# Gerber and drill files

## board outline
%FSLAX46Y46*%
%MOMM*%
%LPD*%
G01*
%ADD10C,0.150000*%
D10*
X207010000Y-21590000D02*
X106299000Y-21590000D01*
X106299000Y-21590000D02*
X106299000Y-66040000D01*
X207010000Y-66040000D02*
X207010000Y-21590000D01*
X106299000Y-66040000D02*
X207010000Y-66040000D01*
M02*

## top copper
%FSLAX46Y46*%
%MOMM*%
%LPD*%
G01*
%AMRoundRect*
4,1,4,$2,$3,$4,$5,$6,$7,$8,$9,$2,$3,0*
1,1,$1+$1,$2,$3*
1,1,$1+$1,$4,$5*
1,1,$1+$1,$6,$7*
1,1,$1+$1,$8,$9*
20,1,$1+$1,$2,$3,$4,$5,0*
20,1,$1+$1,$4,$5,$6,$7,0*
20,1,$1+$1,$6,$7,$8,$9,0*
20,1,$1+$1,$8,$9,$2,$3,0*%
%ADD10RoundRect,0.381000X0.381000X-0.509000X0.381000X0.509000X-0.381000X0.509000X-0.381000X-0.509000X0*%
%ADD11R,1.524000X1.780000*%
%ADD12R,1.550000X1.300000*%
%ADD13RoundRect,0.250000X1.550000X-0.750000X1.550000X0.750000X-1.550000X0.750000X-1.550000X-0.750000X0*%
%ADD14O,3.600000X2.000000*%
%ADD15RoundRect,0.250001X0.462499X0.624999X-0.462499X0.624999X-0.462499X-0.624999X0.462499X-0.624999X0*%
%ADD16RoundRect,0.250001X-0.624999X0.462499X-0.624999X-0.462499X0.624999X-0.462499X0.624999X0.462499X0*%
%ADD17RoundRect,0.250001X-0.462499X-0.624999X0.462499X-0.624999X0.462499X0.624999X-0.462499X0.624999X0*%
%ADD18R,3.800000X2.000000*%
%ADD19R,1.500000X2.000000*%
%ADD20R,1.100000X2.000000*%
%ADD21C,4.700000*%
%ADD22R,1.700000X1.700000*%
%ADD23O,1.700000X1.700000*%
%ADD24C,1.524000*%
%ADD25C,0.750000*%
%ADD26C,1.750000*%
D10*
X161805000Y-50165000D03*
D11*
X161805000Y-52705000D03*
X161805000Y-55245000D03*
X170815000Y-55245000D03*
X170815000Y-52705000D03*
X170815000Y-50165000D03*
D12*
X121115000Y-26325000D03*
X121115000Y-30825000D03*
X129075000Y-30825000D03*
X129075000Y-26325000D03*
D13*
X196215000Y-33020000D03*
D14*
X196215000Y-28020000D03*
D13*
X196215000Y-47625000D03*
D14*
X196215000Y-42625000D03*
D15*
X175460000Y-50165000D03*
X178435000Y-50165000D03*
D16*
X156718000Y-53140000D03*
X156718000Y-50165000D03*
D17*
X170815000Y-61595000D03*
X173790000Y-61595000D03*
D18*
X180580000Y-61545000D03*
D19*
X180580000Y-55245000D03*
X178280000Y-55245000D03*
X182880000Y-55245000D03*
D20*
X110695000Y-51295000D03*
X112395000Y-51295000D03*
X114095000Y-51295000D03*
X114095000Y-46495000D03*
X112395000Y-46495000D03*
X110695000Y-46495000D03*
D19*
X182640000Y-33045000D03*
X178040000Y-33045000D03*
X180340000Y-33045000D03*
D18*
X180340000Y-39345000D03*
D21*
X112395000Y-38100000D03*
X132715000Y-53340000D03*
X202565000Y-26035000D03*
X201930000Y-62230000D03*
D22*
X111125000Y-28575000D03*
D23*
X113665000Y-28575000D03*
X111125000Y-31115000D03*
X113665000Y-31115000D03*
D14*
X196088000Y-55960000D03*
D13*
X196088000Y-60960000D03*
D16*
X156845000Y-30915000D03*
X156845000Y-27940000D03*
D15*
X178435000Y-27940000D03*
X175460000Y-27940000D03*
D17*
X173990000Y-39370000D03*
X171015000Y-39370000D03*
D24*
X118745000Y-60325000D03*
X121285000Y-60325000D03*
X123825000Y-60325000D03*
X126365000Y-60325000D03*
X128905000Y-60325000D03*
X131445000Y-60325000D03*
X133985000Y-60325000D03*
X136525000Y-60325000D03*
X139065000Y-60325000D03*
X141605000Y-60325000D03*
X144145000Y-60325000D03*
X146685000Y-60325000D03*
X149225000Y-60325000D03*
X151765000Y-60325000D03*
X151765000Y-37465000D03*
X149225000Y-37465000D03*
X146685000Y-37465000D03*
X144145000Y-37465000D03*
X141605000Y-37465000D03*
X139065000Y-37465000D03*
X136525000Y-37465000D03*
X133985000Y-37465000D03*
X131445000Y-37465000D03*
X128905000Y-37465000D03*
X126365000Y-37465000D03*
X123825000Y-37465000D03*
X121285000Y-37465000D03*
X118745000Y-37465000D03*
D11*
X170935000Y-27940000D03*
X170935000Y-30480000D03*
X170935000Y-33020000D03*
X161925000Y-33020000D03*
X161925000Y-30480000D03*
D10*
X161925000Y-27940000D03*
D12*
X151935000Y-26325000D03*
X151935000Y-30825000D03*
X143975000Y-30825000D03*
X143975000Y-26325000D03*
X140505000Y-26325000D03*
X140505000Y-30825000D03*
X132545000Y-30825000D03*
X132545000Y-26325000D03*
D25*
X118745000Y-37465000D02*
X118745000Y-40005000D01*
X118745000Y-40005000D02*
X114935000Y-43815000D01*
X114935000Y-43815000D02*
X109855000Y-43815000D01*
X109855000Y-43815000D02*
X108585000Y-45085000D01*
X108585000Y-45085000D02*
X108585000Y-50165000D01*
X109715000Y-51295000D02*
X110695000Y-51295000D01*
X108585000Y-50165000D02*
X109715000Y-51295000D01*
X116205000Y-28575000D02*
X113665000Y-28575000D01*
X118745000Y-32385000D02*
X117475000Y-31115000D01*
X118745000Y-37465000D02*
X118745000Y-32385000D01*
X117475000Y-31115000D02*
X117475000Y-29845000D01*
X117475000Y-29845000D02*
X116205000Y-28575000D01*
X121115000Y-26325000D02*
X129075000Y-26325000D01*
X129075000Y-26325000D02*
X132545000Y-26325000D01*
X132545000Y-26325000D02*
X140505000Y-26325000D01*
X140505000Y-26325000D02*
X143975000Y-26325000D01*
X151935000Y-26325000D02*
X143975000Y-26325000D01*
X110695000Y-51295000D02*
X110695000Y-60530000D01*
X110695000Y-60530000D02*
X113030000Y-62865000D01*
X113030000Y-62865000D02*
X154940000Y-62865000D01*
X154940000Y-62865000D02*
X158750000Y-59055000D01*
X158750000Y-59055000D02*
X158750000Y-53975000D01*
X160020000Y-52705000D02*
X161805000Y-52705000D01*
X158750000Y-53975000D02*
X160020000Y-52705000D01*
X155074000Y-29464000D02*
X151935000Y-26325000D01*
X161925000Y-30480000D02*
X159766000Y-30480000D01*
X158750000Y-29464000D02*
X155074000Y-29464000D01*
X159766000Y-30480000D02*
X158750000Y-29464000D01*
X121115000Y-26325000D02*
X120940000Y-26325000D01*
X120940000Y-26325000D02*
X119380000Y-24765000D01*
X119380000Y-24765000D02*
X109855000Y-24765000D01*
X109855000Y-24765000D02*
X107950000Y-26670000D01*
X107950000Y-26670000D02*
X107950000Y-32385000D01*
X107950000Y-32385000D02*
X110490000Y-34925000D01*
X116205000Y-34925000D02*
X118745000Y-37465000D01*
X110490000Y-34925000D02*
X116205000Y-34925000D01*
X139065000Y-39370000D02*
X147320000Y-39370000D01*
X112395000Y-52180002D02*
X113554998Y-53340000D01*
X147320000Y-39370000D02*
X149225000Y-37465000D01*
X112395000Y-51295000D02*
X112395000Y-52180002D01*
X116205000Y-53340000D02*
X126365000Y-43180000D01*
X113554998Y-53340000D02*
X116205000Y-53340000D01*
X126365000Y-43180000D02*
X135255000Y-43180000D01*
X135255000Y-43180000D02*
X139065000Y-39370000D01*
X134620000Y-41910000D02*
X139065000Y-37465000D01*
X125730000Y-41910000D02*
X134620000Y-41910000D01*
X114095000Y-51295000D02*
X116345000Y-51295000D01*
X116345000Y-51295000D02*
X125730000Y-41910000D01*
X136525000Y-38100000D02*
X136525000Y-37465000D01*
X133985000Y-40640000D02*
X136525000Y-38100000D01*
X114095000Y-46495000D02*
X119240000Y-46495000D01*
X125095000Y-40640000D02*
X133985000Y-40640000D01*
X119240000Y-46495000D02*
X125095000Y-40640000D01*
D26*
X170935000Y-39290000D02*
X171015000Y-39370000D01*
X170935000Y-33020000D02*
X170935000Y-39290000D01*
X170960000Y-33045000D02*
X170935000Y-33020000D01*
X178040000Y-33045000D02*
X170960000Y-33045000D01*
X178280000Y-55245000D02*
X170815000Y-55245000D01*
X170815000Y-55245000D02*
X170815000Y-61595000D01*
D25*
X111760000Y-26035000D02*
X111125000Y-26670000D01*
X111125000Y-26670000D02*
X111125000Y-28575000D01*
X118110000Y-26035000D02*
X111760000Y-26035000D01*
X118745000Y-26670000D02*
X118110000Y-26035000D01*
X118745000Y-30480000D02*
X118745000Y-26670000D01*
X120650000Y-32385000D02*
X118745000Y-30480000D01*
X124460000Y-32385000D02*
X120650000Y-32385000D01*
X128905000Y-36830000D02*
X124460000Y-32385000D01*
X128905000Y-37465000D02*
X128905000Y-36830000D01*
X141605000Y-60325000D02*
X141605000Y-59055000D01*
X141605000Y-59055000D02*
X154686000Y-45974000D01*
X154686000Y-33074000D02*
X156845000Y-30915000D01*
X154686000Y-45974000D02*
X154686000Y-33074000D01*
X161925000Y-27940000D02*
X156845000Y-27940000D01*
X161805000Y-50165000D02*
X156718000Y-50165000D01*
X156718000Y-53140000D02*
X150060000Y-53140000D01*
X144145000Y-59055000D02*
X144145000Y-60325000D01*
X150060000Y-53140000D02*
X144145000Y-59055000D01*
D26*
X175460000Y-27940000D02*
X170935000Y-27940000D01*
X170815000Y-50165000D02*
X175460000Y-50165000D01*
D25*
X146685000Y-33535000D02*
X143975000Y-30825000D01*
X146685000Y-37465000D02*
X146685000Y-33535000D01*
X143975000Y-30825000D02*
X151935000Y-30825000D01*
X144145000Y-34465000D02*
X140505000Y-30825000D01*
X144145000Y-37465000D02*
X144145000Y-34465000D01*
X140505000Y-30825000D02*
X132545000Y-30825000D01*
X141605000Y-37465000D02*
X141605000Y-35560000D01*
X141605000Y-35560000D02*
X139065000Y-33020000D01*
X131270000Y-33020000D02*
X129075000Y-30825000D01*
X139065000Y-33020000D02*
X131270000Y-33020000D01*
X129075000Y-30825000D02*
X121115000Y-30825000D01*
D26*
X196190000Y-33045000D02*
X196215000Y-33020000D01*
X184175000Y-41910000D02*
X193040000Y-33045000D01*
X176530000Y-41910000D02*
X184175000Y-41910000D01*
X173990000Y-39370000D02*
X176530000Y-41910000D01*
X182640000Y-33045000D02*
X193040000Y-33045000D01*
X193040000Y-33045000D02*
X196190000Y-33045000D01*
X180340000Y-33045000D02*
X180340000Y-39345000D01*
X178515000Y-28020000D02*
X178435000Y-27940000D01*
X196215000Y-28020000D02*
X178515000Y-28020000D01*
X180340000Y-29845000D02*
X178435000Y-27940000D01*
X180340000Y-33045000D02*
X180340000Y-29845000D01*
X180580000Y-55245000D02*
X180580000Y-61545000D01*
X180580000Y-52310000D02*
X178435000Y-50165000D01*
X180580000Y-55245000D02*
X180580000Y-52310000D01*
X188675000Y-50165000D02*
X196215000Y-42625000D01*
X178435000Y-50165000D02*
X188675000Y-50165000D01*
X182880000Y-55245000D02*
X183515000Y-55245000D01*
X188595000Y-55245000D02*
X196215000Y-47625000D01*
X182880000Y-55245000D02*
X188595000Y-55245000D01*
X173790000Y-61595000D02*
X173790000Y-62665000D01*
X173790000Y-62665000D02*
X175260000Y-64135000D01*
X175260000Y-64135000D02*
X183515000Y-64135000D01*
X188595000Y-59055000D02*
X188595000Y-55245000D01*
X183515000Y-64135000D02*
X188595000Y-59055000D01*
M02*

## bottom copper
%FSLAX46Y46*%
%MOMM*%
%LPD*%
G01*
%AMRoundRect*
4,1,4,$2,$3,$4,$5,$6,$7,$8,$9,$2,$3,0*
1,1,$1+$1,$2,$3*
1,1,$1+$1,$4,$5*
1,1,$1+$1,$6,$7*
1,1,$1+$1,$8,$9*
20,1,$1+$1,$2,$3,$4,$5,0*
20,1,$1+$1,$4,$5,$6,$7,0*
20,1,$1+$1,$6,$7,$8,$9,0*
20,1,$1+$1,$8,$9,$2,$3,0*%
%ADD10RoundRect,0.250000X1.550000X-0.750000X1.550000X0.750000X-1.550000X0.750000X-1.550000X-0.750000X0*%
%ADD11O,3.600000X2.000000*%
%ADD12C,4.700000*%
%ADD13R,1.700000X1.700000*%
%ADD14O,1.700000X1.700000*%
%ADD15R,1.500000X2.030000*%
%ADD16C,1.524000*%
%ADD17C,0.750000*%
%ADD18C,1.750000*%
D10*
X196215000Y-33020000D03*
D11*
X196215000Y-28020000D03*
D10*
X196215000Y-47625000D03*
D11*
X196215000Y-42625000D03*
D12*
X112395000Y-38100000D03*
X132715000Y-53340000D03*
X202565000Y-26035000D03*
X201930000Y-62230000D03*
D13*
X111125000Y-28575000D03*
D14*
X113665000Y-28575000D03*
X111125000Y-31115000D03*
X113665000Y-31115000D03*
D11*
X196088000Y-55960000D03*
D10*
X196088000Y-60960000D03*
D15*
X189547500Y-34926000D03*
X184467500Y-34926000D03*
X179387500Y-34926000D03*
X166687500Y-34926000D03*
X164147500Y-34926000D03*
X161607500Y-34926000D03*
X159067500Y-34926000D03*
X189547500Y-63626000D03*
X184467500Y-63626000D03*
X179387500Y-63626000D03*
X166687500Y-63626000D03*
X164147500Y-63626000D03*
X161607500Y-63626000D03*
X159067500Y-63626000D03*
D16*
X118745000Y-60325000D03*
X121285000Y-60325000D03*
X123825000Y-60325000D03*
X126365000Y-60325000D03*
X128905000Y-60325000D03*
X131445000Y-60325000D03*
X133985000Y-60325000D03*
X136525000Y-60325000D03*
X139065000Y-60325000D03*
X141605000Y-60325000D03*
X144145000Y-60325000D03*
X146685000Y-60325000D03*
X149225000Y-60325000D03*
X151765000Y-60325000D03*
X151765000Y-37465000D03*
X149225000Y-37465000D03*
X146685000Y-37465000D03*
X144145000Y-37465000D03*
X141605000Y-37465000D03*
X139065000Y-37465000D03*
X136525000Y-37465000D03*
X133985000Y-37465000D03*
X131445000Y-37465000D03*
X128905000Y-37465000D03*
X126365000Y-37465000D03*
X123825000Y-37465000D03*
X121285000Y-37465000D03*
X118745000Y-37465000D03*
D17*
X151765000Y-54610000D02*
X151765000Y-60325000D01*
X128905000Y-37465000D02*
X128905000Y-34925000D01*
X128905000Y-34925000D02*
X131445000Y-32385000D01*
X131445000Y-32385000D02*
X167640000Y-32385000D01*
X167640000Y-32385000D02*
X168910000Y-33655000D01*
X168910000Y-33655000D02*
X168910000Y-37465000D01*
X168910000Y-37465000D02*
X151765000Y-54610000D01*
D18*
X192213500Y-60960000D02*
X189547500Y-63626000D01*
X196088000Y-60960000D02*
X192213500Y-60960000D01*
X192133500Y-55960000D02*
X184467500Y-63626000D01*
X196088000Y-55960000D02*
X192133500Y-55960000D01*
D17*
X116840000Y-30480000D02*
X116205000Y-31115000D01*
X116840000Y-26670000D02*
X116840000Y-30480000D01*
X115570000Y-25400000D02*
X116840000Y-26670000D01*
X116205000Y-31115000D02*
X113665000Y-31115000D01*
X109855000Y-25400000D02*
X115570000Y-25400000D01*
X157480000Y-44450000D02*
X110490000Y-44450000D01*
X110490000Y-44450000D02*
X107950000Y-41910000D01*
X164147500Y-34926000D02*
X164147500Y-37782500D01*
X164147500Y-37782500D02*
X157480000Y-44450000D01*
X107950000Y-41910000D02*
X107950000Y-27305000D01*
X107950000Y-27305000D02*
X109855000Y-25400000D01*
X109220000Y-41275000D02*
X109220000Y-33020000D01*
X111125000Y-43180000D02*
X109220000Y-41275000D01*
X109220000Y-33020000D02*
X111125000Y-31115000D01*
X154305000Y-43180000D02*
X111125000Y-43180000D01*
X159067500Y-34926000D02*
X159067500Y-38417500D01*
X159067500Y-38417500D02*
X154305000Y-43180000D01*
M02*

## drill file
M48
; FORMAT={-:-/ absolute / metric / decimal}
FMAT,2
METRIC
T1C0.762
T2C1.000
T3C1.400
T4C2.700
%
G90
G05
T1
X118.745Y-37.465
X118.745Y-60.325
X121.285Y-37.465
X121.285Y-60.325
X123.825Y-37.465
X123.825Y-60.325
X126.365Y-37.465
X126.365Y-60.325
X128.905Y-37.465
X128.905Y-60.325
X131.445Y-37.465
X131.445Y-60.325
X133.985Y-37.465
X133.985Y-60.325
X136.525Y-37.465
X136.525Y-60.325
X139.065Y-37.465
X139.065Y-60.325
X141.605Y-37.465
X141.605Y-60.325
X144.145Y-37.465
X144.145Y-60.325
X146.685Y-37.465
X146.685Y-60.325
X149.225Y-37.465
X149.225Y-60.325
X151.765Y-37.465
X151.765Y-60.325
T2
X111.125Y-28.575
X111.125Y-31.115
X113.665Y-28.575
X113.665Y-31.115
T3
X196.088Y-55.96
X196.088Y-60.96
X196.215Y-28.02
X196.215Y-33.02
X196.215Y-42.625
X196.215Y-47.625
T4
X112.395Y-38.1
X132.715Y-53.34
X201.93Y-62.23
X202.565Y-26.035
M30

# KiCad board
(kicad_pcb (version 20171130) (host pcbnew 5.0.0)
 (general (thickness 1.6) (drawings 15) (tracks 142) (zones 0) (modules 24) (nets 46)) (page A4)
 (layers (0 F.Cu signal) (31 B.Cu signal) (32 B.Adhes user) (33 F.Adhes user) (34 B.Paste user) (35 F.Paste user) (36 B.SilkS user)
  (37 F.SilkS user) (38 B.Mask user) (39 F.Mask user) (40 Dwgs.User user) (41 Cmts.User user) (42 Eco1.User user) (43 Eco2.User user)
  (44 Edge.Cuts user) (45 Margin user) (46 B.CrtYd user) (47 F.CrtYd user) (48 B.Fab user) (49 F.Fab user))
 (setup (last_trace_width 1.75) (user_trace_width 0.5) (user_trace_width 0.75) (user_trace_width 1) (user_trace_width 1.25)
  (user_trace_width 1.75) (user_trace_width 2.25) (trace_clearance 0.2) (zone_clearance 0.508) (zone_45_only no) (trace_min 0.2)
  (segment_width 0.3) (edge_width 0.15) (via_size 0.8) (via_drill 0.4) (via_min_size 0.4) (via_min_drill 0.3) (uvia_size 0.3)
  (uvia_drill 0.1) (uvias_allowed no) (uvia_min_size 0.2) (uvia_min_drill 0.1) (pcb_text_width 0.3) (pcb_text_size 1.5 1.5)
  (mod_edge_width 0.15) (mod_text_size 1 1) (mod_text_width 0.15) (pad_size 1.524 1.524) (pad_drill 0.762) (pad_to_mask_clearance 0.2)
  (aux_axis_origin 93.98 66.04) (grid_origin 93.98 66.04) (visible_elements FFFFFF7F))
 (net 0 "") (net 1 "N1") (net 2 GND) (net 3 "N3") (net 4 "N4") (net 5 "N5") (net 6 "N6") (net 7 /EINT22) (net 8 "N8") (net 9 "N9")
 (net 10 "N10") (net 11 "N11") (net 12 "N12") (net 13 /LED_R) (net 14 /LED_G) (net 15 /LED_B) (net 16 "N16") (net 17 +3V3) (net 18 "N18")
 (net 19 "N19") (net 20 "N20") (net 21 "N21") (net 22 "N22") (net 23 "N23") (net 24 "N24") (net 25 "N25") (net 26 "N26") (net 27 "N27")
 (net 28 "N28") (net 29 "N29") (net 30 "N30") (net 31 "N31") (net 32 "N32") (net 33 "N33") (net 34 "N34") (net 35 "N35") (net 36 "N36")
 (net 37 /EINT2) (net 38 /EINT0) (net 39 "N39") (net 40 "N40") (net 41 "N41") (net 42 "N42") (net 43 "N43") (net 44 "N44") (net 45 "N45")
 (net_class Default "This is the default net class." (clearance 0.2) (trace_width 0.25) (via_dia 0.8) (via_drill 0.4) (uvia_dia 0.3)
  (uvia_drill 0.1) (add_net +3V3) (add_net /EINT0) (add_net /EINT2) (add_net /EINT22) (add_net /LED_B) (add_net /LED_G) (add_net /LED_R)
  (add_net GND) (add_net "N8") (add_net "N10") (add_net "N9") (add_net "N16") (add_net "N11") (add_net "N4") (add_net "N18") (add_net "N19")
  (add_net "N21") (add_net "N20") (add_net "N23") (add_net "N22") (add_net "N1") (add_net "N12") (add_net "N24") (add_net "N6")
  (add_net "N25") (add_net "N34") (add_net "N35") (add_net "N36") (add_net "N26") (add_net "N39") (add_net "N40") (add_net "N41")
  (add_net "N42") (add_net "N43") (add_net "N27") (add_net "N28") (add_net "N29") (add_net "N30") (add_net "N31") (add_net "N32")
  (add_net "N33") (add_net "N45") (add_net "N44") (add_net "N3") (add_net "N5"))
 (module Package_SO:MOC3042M (layer F.Cu) (at 166.885 52.705 270)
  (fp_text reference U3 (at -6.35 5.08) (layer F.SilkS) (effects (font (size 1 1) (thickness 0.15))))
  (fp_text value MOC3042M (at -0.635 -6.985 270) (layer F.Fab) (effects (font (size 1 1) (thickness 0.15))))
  (pad 1 smd roundrect (at -2.54 5.08 90) (size 1.78 1.524) (layers F.Cu F.Paste F.Mask) (roundrect_rratio 0.25) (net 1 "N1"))
  (pad 2 smd rect (at 0 5.08 90) (size 1.78 1.524) (layers F.Cu F.Paste F.Mask) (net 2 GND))
  (pad 3 smd rect (at 2.54 5.08 90) (size 1.78 1.524) (layers F.Cu F.Paste F.Mask) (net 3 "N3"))
  (pad 4 smd rect (at 2.54 -3.93 90) (size 1.78 1.524) (layers F.Cu F.Paste F.Mask) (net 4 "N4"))
  (pad 5 smd rect (at 0 -3.93 90) (size 1.78 1.524) (layers F.Cu F.Paste F.Mask) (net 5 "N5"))
  (pad 6 smd rect (at -2.54 -3.93 90) (size 1.78 1.524) (layers F.Cu F.Paste F.Mask) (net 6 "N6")))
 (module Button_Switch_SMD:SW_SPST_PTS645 (layer F.Cu) (at 125.095 28.575 180)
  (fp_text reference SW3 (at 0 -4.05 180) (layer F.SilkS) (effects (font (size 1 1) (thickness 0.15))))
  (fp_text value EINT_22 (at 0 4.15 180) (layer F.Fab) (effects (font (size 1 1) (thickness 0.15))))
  (pad 2 smd rect (at 3.98 2.25 180) (size 1.55 1.3) (layers F.Cu F.Paste F.Mask) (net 2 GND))
  (pad 1 smd rect (at 3.98 -2.25 180) (size 1.55 1.3) (layers F.Cu F.Paste F.Mask) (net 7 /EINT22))
  (pad 1 smd rect (at -3.98 -2.25 180) (size 1.55 1.3) (layers F.Cu F.Paste F.Mask) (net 7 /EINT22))
  (pad 2 smd rect (at -3.98 2.25 180) (size 1.55 1.3) (layers F.Cu F.Paste F.Mask) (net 2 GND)))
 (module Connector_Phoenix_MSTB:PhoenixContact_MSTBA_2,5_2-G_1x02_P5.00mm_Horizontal (layer F.Cu) (at 196.215 33.02 90)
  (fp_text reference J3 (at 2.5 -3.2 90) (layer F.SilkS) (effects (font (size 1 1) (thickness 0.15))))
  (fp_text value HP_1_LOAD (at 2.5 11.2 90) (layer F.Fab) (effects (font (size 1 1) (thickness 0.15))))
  (pad 1 thru_hole roundrect (at 0 0 90) (size 2 3.6) (drill 1.4) (layers *.Cu *.Mask) (roundrect_rratio 0.125) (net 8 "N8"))
  (pad 2 thru_hole oval (at 5 0 90) (size 2 3.6) (drill 1.4) (layers *.Cu *.Mask) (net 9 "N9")))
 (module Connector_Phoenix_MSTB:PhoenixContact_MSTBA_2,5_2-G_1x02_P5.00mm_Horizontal (layer F.Cu) (at 196.215 47.625 90)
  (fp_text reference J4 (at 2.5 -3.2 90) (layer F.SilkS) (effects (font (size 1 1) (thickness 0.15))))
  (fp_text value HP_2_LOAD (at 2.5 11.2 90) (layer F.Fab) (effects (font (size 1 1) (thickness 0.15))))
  (pad 1 thru_hole roundrect (at 0 0 90) (size 2 3.6) (drill 1.4) (layers *.Cu *.Mask) (roundrect_rratio 0.125) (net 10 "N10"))
  (pad 2 thru_hole oval (at 5 0 90) (size 2 3.6) (drill 1.4) (layers *.Cu *.Mask) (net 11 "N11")))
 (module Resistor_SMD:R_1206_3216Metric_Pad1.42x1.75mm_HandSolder (layer F.Cu) (at 176.9475 50.165 180)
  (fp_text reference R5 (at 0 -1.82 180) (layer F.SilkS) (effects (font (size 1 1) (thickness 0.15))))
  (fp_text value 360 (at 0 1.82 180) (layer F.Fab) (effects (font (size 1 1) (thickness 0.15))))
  (pad 2 smd roundrect (at 1.4875 0 180) (size 1.425 1.75) (layers F.Cu F.Paste F.Mask) (roundrect_rratio 0.175439) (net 6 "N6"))
  (pad 1 smd roundrect (at -1.4875 0 180) (size 1.425 1.75) (layers F.Cu F.Paste F.Mask) (roundrect_rratio 0.175439) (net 11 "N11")))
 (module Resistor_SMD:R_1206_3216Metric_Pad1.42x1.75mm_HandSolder (layer F.Cu) (at 156.718 51.6525 270)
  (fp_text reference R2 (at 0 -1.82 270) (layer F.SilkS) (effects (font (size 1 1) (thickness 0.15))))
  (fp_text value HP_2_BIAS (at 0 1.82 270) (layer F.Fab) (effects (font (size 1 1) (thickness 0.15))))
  (pad 2 smd roundrect (at 1.4875 0 270) (size 1.425 1.75) (layers F.Cu F.Paste F.Mask) (roundrect_rratio 0.175439) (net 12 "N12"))
  (pad 1 smd roundrect (at -1.4875 0 270) (size 1.425 1.75) (layers F.Cu F.Paste F.Mask) (roundrect_rratio 0.175439) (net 1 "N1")))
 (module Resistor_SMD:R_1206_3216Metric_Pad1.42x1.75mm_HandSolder (layer F.Cu) (at 172.3025 61.595)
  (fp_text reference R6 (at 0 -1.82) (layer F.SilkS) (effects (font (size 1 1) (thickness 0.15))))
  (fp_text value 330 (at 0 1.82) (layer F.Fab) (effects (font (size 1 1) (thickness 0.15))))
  (pad 1 smd roundrect (at -1.4875 0) (size 1.425 1.75) (layers F.Cu F.Paste F.Mask) (roundrect_rratio 0.175439) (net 4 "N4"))
  (pad 2 smd roundrect (at 1.4875 0) (size 1.425 1.75) (layers F.Cu F.Paste F.Mask) (roundrect_rratio 0.175439) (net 10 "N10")))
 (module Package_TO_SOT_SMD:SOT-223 (layer F.Cu) (at 180.58 58.395 270)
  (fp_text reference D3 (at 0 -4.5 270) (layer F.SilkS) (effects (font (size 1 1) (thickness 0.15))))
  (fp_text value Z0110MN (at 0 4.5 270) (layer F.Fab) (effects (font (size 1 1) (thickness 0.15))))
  (pad 4 smd rect (at 3.15 0 270) (size 2 3.8) (layers F.Cu F.Paste F.Mask) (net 11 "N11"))
  (pad 2 smd rect (at -3.15 0 270) (size 2 1.5) (layers F.Cu F.Paste F.Mask) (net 11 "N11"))
  (pad 3 smd rect (at -3.15 2.3 270) (size 2 1.5) (layers F.Cu F.Paste F.Mask) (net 4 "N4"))
  (pad 1 smd rect (at -3.15 -2.3 270) (size 2 1.5) (layers F.Cu F.Paste F.Mask) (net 10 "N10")))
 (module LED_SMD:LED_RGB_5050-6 (layer F.Cu) (at 112.395 48.895 90)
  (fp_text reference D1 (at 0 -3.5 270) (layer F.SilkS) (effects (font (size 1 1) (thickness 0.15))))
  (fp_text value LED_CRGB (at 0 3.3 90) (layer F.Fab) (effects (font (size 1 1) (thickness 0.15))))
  (pad 1 smd rect (at -2.4 -1.7 180) (size 1.1 2) (layers F.Cu F.Paste F.Mask) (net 2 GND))
  (pad 2 smd rect (at -2.4 0 180) (size 1.1 2) (layers F.Cu F.Paste F.Mask) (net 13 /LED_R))
  (pad 3 smd rect (at -2.4 1.7 180) (size 1.1 2) (layers F.Cu F.Paste F.Mask) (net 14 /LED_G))
  (pad 4 smd rect (at 2.4 1.7 180) (size 1.1 2) (layers F.Cu F.Paste F.Mask) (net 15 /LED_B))
  (pad 5 smd rect (at 2.4 0 180) (size 1.1 2) (layers F.Cu F.Paste F.Mask))
  (pad 6 smd rect (at 2.4 -1.7 180) (size 1.1 2) (layers F.Cu F.Paste F.Mask)))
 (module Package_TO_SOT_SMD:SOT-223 (layer F.Cu) (at 180.34 36.195 270)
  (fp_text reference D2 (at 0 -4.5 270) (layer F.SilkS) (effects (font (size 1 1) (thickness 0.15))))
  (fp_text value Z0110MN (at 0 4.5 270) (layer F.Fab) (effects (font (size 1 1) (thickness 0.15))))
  (pad 1 smd rect (at -3.15 -2.3 270) (size 2 1.5) (layers F.Cu F.Paste F.Mask) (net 8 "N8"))
  (pad 3 smd rect (at -3.15 2.3 270) (size 2 1.5) (layers F.Cu F.Paste F.Mask) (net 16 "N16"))
  (pad 2 smd rect (at -3.15 0 270) (size 2 1.5) (layers F.Cu F.Paste F.Mask) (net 9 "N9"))
  (pad 4 smd rect (at 3.15 0 270) (size 2 3.8) (layers F.Cu F.Paste F.Mask) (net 9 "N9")))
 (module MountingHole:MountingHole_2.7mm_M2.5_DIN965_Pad (layer F.Cu) (at 112.395 38.1)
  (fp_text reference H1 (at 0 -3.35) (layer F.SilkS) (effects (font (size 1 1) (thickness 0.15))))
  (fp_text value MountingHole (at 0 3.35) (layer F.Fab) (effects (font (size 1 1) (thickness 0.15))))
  (pad 1 thru_hole circle (at 0 0) (size 4.7 4.7) (drill 2.7) (layers *.Cu *.Mask)))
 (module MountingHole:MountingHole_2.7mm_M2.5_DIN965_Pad (layer F.Cu) (at 132.715 53.34)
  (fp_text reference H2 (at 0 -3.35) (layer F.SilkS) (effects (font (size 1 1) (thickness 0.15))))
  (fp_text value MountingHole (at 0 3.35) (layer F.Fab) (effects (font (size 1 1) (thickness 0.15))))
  (pad 1 thru_hole circle (at 0 0) (size 4.7 4.7) (drill 2.7) (layers *.Cu *.Mask)))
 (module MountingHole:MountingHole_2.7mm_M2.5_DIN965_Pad (layer F.Cu) (at 202.565 26.035)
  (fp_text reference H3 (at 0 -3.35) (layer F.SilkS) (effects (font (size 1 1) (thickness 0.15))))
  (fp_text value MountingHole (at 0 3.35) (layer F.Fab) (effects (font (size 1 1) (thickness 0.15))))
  (pad 1 thru_hole circle (at 0 0) (size 4.7 4.7) (drill 2.7) (layers *.Cu *.Mask)))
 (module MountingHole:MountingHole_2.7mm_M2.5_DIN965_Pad (layer F.Cu) (at 201.93 62.23)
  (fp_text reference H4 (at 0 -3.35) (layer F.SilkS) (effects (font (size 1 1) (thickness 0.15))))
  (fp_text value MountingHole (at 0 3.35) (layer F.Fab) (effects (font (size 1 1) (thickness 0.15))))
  (pad 1 thru_hole circle (at 0 0) (size 4.7 4.7) (drill 2.7) (layers *.Cu *.Mask)))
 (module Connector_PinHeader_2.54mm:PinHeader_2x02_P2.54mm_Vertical (layer F.Cu) (at 111.125 28.575)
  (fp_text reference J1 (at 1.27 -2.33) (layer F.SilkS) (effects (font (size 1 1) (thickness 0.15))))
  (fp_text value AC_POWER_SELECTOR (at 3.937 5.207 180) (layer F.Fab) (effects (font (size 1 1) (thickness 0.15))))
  (pad 1 thru_hole rect (at 0 0) (size 1.7 1.7) (drill 1) (layers *.Cu *.Mask) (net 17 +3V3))
  (pad 2 thru_hole oval (at 2.54 0) (size 1.7 1.7) (drill 1) (layers *.Cu *.Mask) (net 2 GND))
  (pad 3 thru_hole oval (at 0 2.54) (size 1.7 1.7) (drill 1) (layers *.Cu *.Mask) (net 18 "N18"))
  (pad 4 thru_hole oval (at 2.54 2.54) (size 1.7 1.7) (drill 1) (layers *.Cu *.Mask) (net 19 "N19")))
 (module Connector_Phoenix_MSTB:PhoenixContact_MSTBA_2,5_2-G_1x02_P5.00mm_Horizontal (layer F.Cu) (at 196.088 60.96 90)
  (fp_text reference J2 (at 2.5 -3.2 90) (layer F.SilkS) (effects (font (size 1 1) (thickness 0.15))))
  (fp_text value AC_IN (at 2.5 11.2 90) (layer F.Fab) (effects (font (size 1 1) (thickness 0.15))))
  (pad 2 thru_hole oval (at 5 0 90) (size 2 3.6) (drill 1.4) (layers *.Cu *.Mask) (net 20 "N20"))
  (pad 1 thru_hole roundrect (at 0 0 90) (size 2 3.6) (drill 1.4) (layers *.Cu *.Mask) (roundrect_rratio 0.125) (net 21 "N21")))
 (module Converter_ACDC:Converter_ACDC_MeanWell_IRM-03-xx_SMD (layer B.Cu) (at 174.3075 49.276 90)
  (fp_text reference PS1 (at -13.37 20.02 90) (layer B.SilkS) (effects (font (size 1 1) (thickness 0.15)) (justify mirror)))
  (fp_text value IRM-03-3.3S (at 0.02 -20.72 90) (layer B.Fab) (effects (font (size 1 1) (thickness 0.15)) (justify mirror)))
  (pad 26 smd rect (at 14.35 15.24 180) (size 1.5 2.03) (layers B.Cu B.Paste B.Mask))
  (pad 24 smd rect (at 14.35 10.16 180) (size 1.5 2.03) (layers B.Cu B.Paste B.Mask))
  (pad 22 smd rect (at 14.35 5.08 180) (size 1.5 2.03) (layers B.Cu B.Paste B.Mask))
  (pad 17 smd rect (at 14.35 -7.62 180) (size 1.5 2.03) (layers B.Cu B.Paste B.Mask))
  (pad 16 smd rect (at 14.35 -10.16 180) (size 1.5 2.03) (layers B.Cu B.Paste B.Mask) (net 19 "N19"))
  (pad 15 smd rect (at 14.35 -12.7 180) (size 1.5 2.03) (layers B.Cu B.Paste B.Mask))
  (pad 14 smd rect (at 14.35 -15.24 180) (size 1.5 2.03) (layers B.Cu B.Paste B.Mask) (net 18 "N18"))
  (pad 1 smd rect (at -14.35 15.24 180) (size 1.5 2.03) (layers B.Cu B.Paste B.Mask) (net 21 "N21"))
  (pad 3 smd rect (at -14.35 10.16 180) (size 1.5 2.03) (layers B.Cu B.Paste B.Mask) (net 20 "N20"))
  (pad 5 smd rect (at -14.35 5.08 180) (size 1.5 2.03) (layers B.Cu B.Paste B.Mask))
  (pad 10 smd rect (at -14.35 -7.62 180) (size 1.5 2.03) (layers B.Cu B.Paste B.Mask))
  (pad 11 smd rect (at -14.35 -10.16 180) (size 1.5 2.03) (layers B.Cu B.Paste B.Mask))
  (pad 12 smd rect (at -14.35 -12.7 180) (size 1.5 2.03) (layers B.Cu B.Paste B.Mask))
  (pad 13 smd rect (at -14.35 -15.24 180) (size 1.5 2.03) (layers B.Cu B.Paste B.Mask)))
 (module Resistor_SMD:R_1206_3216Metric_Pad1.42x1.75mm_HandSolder (layer F.Cu) (at 156.845 29.4275 270)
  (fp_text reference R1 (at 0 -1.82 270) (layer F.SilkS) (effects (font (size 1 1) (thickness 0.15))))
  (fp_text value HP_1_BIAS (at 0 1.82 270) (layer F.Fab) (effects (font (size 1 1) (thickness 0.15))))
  (pad 2 smd roundrect (at 1.4875 0 270) (size 1.425 1.75) (layers F.Cu F.Paste F.Mask) (roundrect_rratio 0.175439) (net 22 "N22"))
  (pad 1 smd roundrect (at -1.4875 0 270) (size 1.425 1.75) (layers F.Cu F.Paste F.Mask) (roundrect_rratio 0.175439) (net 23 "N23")))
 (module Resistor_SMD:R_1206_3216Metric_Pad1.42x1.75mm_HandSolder (layer F.Cu) (at 176.9475 27.94 180)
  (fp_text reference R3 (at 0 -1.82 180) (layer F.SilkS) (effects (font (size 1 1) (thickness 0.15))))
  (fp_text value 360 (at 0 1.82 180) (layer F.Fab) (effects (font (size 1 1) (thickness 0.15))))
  (pad 1 smd roundrect (at -1.4875 0 180) (size 1.425 1.75) (layers F.Cu F.Paste F.Mask) (roundrect_rratio 0.175439) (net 9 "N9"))
  (pad 2 smd roundrect (at 1.4875 0 180) (size 1.425 1.75) (layers F.Cu F.Paste F.Mask) (roundrect_rratio 0.175439) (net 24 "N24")))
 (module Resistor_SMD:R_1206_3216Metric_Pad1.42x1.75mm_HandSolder (layer F.Cu) (at 172.5025 39.37)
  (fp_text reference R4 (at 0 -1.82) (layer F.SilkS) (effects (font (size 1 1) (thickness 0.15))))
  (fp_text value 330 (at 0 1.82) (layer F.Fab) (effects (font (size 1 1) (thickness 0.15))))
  (pad 2 smd roundrect (at 1.4875 0) (size 1.425 1.75) (layers F.Cu F.Paste F.Mask) (roundrect_rratio 0.175439) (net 8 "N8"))
  (pad 1 smd roundrect (at -1.4875 0) (size 1.425 1.75) (layers F.Cu F.Paste F.Mask) (roundrect_rratio 0.175439) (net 16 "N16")))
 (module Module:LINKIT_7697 (layer F.Cu) (at 151.765 37.465 180)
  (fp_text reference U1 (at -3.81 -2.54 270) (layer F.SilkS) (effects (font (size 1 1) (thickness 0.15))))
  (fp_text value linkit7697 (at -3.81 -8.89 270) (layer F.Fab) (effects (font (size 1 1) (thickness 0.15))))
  (pad 1 thru_hole circle (at 33.02 -22.86 180) (size 1.524 1.524) (drill 0.762) (layers *.Cu *.Mask) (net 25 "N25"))
  (pad 2 thru_hole circle (at 30.48 -22.86 180) (size 1.524 1.524) (drill 0.762) (layers *.Cu *.Mask) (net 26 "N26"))
  (pad 3 thru_hole circle (at 27.94 -22.86 180) (size 1.524 1.524) (drill 0.762) (layers *.Cu *.Mask) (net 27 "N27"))
  (pad 4 thru_hole circle (at 25.4 -22.86 180) (size 1.524 1.524) (drill 0.762) (layers *.Cu *.Mask) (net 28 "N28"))
  (pad 5 thru_hole circle (at 22.86 -22.86 180) (size 1.524 1.524) (drill 0.762) (layers *.Cu *.Mask) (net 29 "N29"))
  (pad 6 thru_hole circle (at 20.32 -22.86 180) (size 1.524 1.524) (drill 0.762) (layers *.Cu *.Mask) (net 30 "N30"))
  (pad 7 thru_hole circle (at 17.78 -22.86 180) (size 1.524 1.524) (drill 0.762) (layers *.Cu *.Mask) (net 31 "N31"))
  (pad 8 thru_hole circle (at 15.24 -22.86 180) (size 1.524 1.524) (drill 0.762) (layers *.Cu *.Mask) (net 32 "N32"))
  (pad 9 thru_hole circle (at 12.7 -22.86 180) (size 1.524 1.524) (drill 0.762) (layers *.Cu *.Mask) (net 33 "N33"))
  (pad 10 thru_hole circle (at 10.16 -22.86 180) (size 1.524 1.524) (drill 0.762) (layers *.Cu *.Mask) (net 22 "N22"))
  (pad 11 thru_hole circle (at 7.62 -22.86 180) (size 1.524 1.524) (drill 0.762) (layers *.Cu *.Mask) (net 12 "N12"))
  (pad 12 thru_hole circle (at 5.08 -22.86 180) (size 1.524 1.524) (drill 0.762) (layers *.Cu *.Mask) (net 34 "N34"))
  (pad 13 thru_hole circle (at 2.54 -22.86 180) (size 1.524 1.524) (drill 0.762) (layers *.Cu *.Mask) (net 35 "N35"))
  (pad 14 thru_hole circle (at 0 -22.86 180) (size 1.524 1.524) (drill 0.762) (layers *.Cu *.Mask) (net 17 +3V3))
  (pad 15 thru_hole circle (at 0 0 180) (size 1.524 1.524) (drill 0.762) (layers *.Cu *.Mask) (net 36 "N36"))
  (pad 16 thru_hole circle (at 2.54 0 180) (size 1.524 1.524) (drill 0.762) (layers *.Cu *.Mask) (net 13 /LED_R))
  (pad 17 thru_hole circle (at 5.08 0 180) (size 1.524 1.524) (drill 0.762) (layers *.Cu *.Mask) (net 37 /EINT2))
  (pad 18 thru_hole circle (at 7.62 0 180) (size 1.524 1.524) (drill 0.762) (layers *.Cu *.Mask) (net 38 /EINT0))
  (pad 19 thru_hole circle (at 10.16 0 180) (size 1.524 1.524) (drill 0.762) (layers *.Cu *.Mask) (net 7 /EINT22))
  (pad 20 thru_hole circle (at 12.7 0 180) (size 1.524 1.524) (drill 0.762) (layers *.Cu *.Mask) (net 14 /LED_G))
  (pad 21 thru_hole circle (at 15.24 0 180) (size 1.524 1.524) (drill 0.762) (layers *.Cu *.Mask) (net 15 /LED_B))
  (pad 22 thru_hole circle (at 17.78 0 180) (size 1.524 1.524) (drill 0.762) (layers *.Cu *.Mask) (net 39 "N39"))
  (pad 23 thru_hole circle (at 20.32 0 180) (size 1.524 1.524) (drill 0.762) (layers *.Cu *.Mask) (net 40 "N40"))
  (pad 24 thru_hole circle (at 22.86 0 180) (size 1.524 1.524) (drill 0.762) (layers *.Cu *.Mask) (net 17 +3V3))
  (pad 25 thru_hole circle (at 25.4 0 180) (size 1.524 1.524) (drill 0.762) (layers *.Cu *.Mask) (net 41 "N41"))
  (pad 26 thru_hole circle (at 27.94 0 180) (size 1.524 1.524) (drill 0.762) (layers *.Cu *.Mask) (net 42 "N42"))
  (pad 27 thru_hole circle (at 30.48 0 180) (size 1.524 1.524) (drill 0.762) (layers *.Cu *.Mask) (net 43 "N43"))
  (pad 28 thru_hole circle (at 33.02 0 180) (size 1.524 1.524) (drill 0.762) (layers *.Cu *.Mask) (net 2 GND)))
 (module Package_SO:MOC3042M (layer F.Cu) (at 167.005 30.48 270)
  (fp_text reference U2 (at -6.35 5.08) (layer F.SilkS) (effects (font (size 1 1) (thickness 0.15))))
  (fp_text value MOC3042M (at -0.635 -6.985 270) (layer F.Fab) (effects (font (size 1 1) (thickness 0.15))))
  (pad 6 smd rect (at -2.54 -3.93 90) (size 1.78 1.524) (layers F.Cu F.Paste F.Mask) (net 24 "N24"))
  (pad 5 smd rect (at 0 -3.93 90) (size 1.78 1.524) (layers F.Cu F.Paste F.Mask) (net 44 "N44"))
  (pad 4 smd rect (at 2.54 -3.93 90) (size 1.78 1.524) (layers F.Cu F.Paste F.Mask) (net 16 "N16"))
  (pad 3 smd rect (at 2.54 5.08 90) (size 1.78 1.524) (layers F.Cu F.Paste F.Mask) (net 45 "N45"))
  (pad 2 smd rect (at 0 5.08 90) (size 1.78 1.524) (layers F.Cu F.Paste F.Mask) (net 2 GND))
  (pad 1 smd roundrect (at -2.54 5.08 90) (size 1.78 1.524) (layers F.Cu F.Paste F.Mask) (roundrect_rratio 0.25) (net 23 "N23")))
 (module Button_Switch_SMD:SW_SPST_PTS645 (layer F.Cu) (at 147.955 28.575 180)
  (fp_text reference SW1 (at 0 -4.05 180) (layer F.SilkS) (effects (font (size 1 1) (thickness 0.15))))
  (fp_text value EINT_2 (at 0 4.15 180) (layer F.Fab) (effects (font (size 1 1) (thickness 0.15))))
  (pad 2 smd rect (at -3.98 2.25 180) (size 1.55 1.3) (layers F.Cu F.Paste F.Mask) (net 2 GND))
  (pad 1 smd rect (at -3.98 -2.25 180) (size 1.55 1.3) (layers F.Cu F.Paste F.Mask) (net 37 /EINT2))
  (pad 1 smd rect (at 3.98 -2.25 180) (size 1.55 1.3) (layers F.Cu F.Paste F.Mask) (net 37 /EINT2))
  (pad 2 smd rect (at 3.98 2.25 180) (size 1.55 1.3) (layers F.Cu F.Paste F.Mask) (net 2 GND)))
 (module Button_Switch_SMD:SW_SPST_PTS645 (layer F.Cu) (at 136.525 28.575 180)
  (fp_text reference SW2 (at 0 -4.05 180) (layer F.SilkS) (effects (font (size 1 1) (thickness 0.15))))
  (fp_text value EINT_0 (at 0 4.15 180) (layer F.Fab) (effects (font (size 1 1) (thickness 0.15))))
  (pad 2 smd rect (at -3.98 2.25 180) (size 1.55 1.3) (layers F.Cu F.Paste F.Mask) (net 2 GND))
  (pad 1 smd rect (at -3.98 -2.25 180) (size 1.55 1.3) (layers F.Cu F.Paste F.Mask) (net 38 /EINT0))
  (pad 1 smd rect (at 3.98 -2.25 180) (size 1.55 1.3) (layers F.Cu F.Paste F.Mask) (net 38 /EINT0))
  (pad 2 smd rect (at 3.98 2.25 180) (size 1.55 1.3) (layers F.Cu F.Paste F.Mask) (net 2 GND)))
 (gr_line (start 207.01 21.59) (end 106.299 21.59) (layer Edge.Cuts) (width 0.15))
 (gr_line (start 106.299 21.59) (end 106.299 66.04) (layer Edge.Cuts) (width 0.15))
 (gr_line (start 207.01 66.04) (end 207.01 21.59) (layer Edge.Cuts) (width 0.15))
 (gr_line (start 106.299 66.04) (end 207.01 66.04) (layer Edge.Cuts) (width 0.15))
 (segment (start 118.745 37.465) (end 118.745 40.005) (width 0.75) (layer F.Cu) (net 2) (status 10))
 (segment (start 118.745 40.005) (end 114.935 43.815) (width 0.75) (layer F.Cu) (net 2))
 (segment (start 114.935 43.815) (end 109.855 43.815) (width 0.75) (layer F.Cu) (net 2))
 (segment (start 109.855 43.815) (end 108.585 45.085) (width 0.75) (layer F.Cu) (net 2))
 (segment (start 108.585 45.085) (end 108.585 50.165) (width 0.75) (layer F.Cu) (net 2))
 (segment (start 109.715 51.295) (end 110.695 51.295) (width 0.75) (layer F.Cu) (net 2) (status 20))
 (segment (start 108.585 50.165) (end 109.715 51.295) (width 0.75) (layer F.Cu) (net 2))
 (segment (start 116.205 28.575) (end 113.665 28.575) (width 0.75) (layer F.Cu) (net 2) (status 20))
 (segment (start 118.745 32.385) (end 117.475 31.115) (width 0.75) (layer F.Cu) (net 2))
 (segment (start 118.745 37.465) (end 118.745 32.385) (width 0.75) (layer F.Cu) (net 2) (status 10))
 (segment (start 117.475 31.115) (end 117.475 29.845) (width 0.75) (layer F.Cu) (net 2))
 (segment (start 117.475 29.845) (end 116.205 28.575) (width 0.75) (layer F.Cu) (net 2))
 (segment (start 121.115 26.325) (end 129.075 26.325) (width 0.75) (layer F.Cu) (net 2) (status 30))
 (segment (start 129.075 26.325) (end 132.545 26.325) (width 0.75) (layer F.Cu) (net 2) (status 30))
 (segment (start 132.545 26.325) (end 140.505 26.325) (width 0.75) (layer F.Cu) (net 2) (status 30))
 (segment (start 140.505 26.325) (end 143.975 26.325) (width 0.75) (layer F.Cu) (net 2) (status 30))
 (segment (start 151.935 26.325) (end 143.975 26.325) (width 0.75) (layer F.Cu) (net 2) (status 30))
 (segment (start 110.695 51.295) (end 110.695 60.53) (width 0.75) (layer F.Cu) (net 2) (status 10))
 (segment (start 110.695 60.53) (end 113.03 62.865) (width 0.75) (layer F.Cu) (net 2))
 (segment (start 113.03 62.865) (end 154.94 62.865) (width 0.75) (layer F.Cu) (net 2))
 (segment (start 154.94 62.865) (end 158.75 59.055) (width 0.75) (layer F.Cu) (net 2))
 (segment (start 158.75 59.055) (end 158.75 53.975) (width 0.75) (layer F.Cu) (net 2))
 (segment (start 160.02 52.705) (end 161.805 52.705) (width 0.75) (layer F.Cu) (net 2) (status 20))
 (segment (start 158.75 53.975) (end 160.02 52.705) (width 0.75) (layer F.Cu) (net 2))
 (segment (start 155.074 29.464) (end 151.935 26.325) (width 0.75) (layer F.Cu) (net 2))
 (segment (start 161.925 30.48) (end 159.766 30.48) (width 0.75) (layer F.Cu) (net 2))
 (segment (start 158.75 29.464) (end 155.074 29.464) (width 0.75) (layer F.Cu) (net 2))
 (segment (start 159.766 30.48) (end 158.75 29.464) (width 0.75) (layer F.Cu) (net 2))
 (segment (start 121.115 26.325) (end 120.94 26.325) (width 0.75) (layer F.Cu) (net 2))
 (segment (start 120.94 26.325) (end 119.38 24.765) (width 0.75) (layer F.Cu) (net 2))
 (segment (start 119.38 24.765) (end 109.855 24.765) (width 0.75) (layer F.Cu) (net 2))
 (segment (start 109.855 24.765) (end 107.95 26.67) (width 0.75) (layer F.Cu) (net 2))
 (segment (start 107.95 26.67) (end 107.95 32.385) (width 0.75) (layer F.Cu) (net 2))
 (segment (start 107.95 32.385) (end 110.49 34.925) (width 0.75) (layer F.Cu) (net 2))
 (segment (start 116.205 34.925) (end 118.745 37.465) (width 0.75) (layer F.Cu) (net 2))
 (segment (start 110.49 34.925) (end 116.205 34.925) (width 0.75) (layer F.Cu) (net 2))
 (segment (start 139.065 39.37) (end 147.32 39.37) (width 0.75) (layer F.Cu) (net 13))
 (segment (start 112.395 52.180002) (end 113.554998 53.34) (width 0.75) (layer F.Cu) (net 13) (status 10))
 (segment (start 147.32 39.37) (end 149.225 37.465) (width 0.75) (layer F.Cu) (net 13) (status 20))
 (segment (start 112.395 51.295) (end 112.395 52.180002) (width 0.75) (layer F.Cu) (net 13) (status 30))
 (segment (start 116.205 53.34) (end 126.365 43.18) (width 0.75) (layer F.Cu) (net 13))
 (segment (start 113.554998 53.34) (end 116.205 53.34) (width 0.75) (layer F.Cu) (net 13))
 (segment (start 126.365 43.18) (end 135.255 43.18) (width 0.75) (layer F.Cu) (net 13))
 (segment (start 135.255 43.18) (end 139.065 39.37) (width 0.75) (layer F.Cu) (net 13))
 (segment (start 134.62 41.91) (end 139.065 37.465) (width 0.75) (layer F.Cu) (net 14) (status 20))
 (segment (start 125.73 41.91) (end 134.62 41.91) (width 0.75) (layer F.Cu) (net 14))
 (segment (start 114.095 51.295) (end 116.345 51.295) (width 0.75) (layer F.Cu) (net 14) (status 10))
 (segment (start 116.345 51.295) (end 125.73 41.91) (width 0.75) (layer F.Cu) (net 14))
 (segment (start 136.525 38.1) (end 136.525 37.465) (width 0.75) (layer F.Cu) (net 15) (status 30))
 (segment (start 133.985 40.64) (end 136.525 38.1) (width 0.75) (layer F.Cu) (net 15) (status 20))
 (segment (start 114.095 46.495) (end 119.24 46.495) (width 0.75) (layer F.Cu) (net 15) (status 10))
 (segment (start 125.095 40.64) (end 133.985 40.64) (width 0.75) (layer F.Cu) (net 15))
 (segment (start 119.24 46.495) (end 125.095 40.64) (width 0.75) (layer F.Cu) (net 15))
 (segment (start 170.935 39.29) (end 171.015 39.37) (width 1.75) (layer F.Cu) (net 16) (status 30))
 (segment (start 170.935 33.02) (end 170.935 39.29) (width 1.75) (layer F.Cu) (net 16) (status 30))
 (segment (start 170.96 33.045) (end 170.935 33.02) (width 1.75) (layer F.Cu) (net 16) (status 30))
 (segment (start 178.04 33.045) (end 170.96 33.045) (width 1.75) (layer F.Cu) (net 16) (status 30))
 (segment (start 178.28 55.245) (end 170.815 55.245) (width 1.75) (layer F.Cu) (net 4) (status 30))
 (segment (start 170.815 55.245) (end 170.815 61.595) (width 1.75) (layer F.Cu) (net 4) (status 30))
 (segment (start 111.76 26.035) (end 111.125 26.67) (width 0.75) (layer F.Cu) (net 17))
 (segment (start 111.125 26.67) (end 111.125 28.575) (width 0.75) (layer F.Cu) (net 17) (status 20))
 (segment (start 118.11 26.035) (end 111.76 26.035) (width 0.75) (layer F.Cu) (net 17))
 (segment (start 118.745 26.67) (end 118.11 26.035) (width 0.75) (layer F.Cu) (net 17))
 (segment (start 118.745 30.48) (end 118.745 26.67) (width 0.75) (layer F.Cu) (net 17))
 (segment (start 120.65 32.385) (end 118.745 30.48) (width 0.75) (layer F.Cu) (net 17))
 (segment (start 124.46 32.385) (end 120.65 32.385) (width 0.75) (layer F.Cu) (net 17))
 (segment (start 128.905 36.83) (end 124.46 32.385) (width 0.75) (layer F.Cu) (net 17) (status 10))
 (segment (start 128.905 37.465) (end 128.905 36.83) (width 0.75) (layer F.Cu) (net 17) (status 30))
 (segment (start 151.765 54.61) (end 151.765 60.325) (width 0.75) (layer B.Cu) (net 17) (status 20))
 (segment (start 128.905 37.465) (end 128.905 34.925) (width 0.75) (layer B.Cu) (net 17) (status 10))
 (segment (start 128.905 34.925) (end 131.445 32.385) (width 0.75) (layer B.Cu) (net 17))
 (segment (start 131.445 32.385) (end 167.64 32.385) (width 0.75) (layer B.Cu) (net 17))
 (segment (start 167.64 32.385) (end 168.91 33.655) (width 0.75) (layer B.Cu) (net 17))
 (segment (start 168.91 33.655) (end 168.91 37.465) (width 0.75) (layer B.Cu) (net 17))
 (segment (start 168.91 37.465) (end 151.765 54.61) (width 0.75) (layer B.Cu) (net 17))
 (segment (start 192.2135 60.96) (end 189.5475 63.626) (width 1.75) (layer B.Cu) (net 21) (status 20))
 (segment (start 196.088 60.96) (end 192.2135 60.96) (width 1.75) (layer B.Cu) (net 21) (status 10))
 (segment (start 192.1335 55.96) (end 184.4675 63.626) (width 1.75) (layer B.Cu) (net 20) (status 20))
 (segment (start 196.088 55.96) (end 192.1335 55.96) (width 1.75) (layer B.Cu) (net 20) (status 10))
 (segment (start 116.84 30.48) (end 116.205 31.115) (width 0.75) (layer B.Cu) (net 19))
 (segment (start 116.84 26.67) (end 116.84 30.48) (width 0.75) (layer B.Cu) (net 19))
 (segment (start 115.57 25.4) (end 116.84 26.67) (width 0.75) (layer B.Cu) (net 19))
 (segment (start 116.205 31.115) (end 113.665 31.115) (width 0.75) (layer B.Cu) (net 19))
 (segment (start 109.855 25.4) (end 115.57 25.4) (width 0.75) (layer B.Cu) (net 19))
 (segment (start 157.48 44.45) (end 110.49 44.45) (width 0.75) (layer B.Cu) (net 19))
 (segment (start 110.49 44.45) (end 107.95 41.91) (width 0.75) (layer B.Cu) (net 19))
 (segment (start 164.1475 34.926) (end 164.1475 37.7825) (width 0.75) (layer B.Cu) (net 19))
 (segment (start 164.1475 37.7825) (end 157.48 44.45) (width 0.75) (layer B.Cu) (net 19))
 (segment (start 107.95 41.91) (end 107.95 27.305) (width 0.75) (layer B.Cu) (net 19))
 (segment (start 107.95 27.305) (end 109.855 25.4) (width 0.75) (layer B.Cu) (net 19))
 (segment (start 109.22 41.275) (end 109.22 33.02) (width 0.75) (layer B.Cu) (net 18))
 (segment (start 111.125 43.18) (end 109.22 41.275) (width 0.75) (layer B.Cu) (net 18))
 (segment (start 109.22 33.02) (end 111.125 31.115) (width 0.75) (layer B.Cu) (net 18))
 (segment (start 154.305 43.18) (end 111.125 43.18) (width 0.75) (layer B.Cu) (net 18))
 (segment (start 159.0675 34.926) (end 159.0675 38.4175) (width 0.75) (layer B.Cu) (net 18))
 (segment (start 159.0675 38.4175) (end 154.305 43.18) (width 0.75) (layer B.Cu) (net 18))
 (segment (start 141.605 60.325) (end 141.605 59.055) (width 0.75) (layer F.Cu) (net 22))
 (segment (start 141.605 59.055) (end 154.686 45.974) (width 0.75) (layer F.Cu) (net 22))
 (segment (start 154.686 33.074) (end 156.845 30.915) (width 0.75) (layer F.Cu) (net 22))
 (segment (start 154.686 45.974) (end 154.686 33.074) (width 0.75) (layer F.Cu) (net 22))
 (segment (start 161.925 27.94) (end 156.845 27.94) (width 0.75) (layer F.Cu) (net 23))
 (segment (start 161.805 50.165) (end 156.718 50.165) (width 0.75) (layer F.Cu) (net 1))
 (segment (start 156.718 53.14) (end 150.06 53.14) (width 0.75) (layer F.Cu) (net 12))
 (segment (start 144.145 59.055) (end 144.145 60.325) (width 0.75) (layer F.Cu) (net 12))
 (segment (start 150.06 53.14) (end 144.145 59.055) (width 0.75) (layer F.Cu) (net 12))
 (segment (start 175.46 27.94) (end 170.935 27.94) (width 1.75) (layer F.Cu) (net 24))
 (segment (start 170.815 50.165) (end 175.46 50.165) (width 1.75) (layer F.Cu) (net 6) (status 30))
 (segment (start 146.685 33.535) (end 143.975 30.825) (width 0.75) (layer F.Cu) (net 37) (status 20))
 (segment (start 146.685 37.465) (end 146.685 33.535) (width 0.75) (layer F.Cu) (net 37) (status 10))
 (segment (start 143.975 30.825) (end 151.935 30.825) (width 0.75) (layer F.Cu) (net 37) (status 30))
 (segment (start 144.145 34.465) (end 140.505 30.825) (width 0.75) (layer F.Cu) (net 38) (status 20))
 (segment (start 144.145 37.465) (end 144.145 34.465) (width 0.75) (layer F.Cu) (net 38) (status 10))
 (segment (start 140.505 30.825) (end 132.545 30.825) (width 0.75) (layer F.Cu) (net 38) (status 30))
 (segment (start 141.605 37.465) (end 141.605 35.56) (width 0.75) (layer F.Cu) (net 7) (status 10))
 (segment (start 141.605 35.56) (end 139.065 33.02) (width 0.75) (layer F.Cu) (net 7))
 (segment (start 131.27 33.02) (end 129.075 30.825) (width 0.75) (layer F.Cu) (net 7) (status 20))
 (segment (start 139.065 33.02) (end 131.27 33.02) (width 0.75) (layer F.Cu) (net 7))
 (segment (start 129.075 30.825) (end 121.115 30.825) (width 0.75) (layer F.Cu) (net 7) (status 30))
 (segment (start 196.19 33.045) (end 196.215 33.02) (width 1.75) (layer F.Cu) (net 8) (status 30))
 (segment (start 184.175 41.91) (end 193.04 33.045) (width 1.75) (layer F.Cu) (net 8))
 (segment (start 176.53 41.91) (end 184.175 41.91) (width 1.75) (layer F.Cu) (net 8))
 (segment (start 173.99 39.37) (end 176.53 41.91) (width 1.75) (layer F.Cu) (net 8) (status 10))
 (segment (start 182.64 33.045) (end 193.04 33.045) (width 1.75) (layer F.Cu) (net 8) (status 10))
 (segment (start 193.04 33.045) (end 196.19 33.045) (width 1.75) (layer F.Cu) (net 8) (status 20))
 (segment (start 180.34 33.045) (end 180.34 39.345) (width 1.75) (layer F.Cu) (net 9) (status 30))
 (segment (start 178.515 28.02) (end 178.435 27.94) (width 1.75) (layer F.Cu) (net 9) (status 30))
 (segment (start 196.215 28.02) (end 178.515 28.02) (width 1.75) (layer F.Cu) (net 9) (status 30))
 (segment (start 180.34 29.845) (end 178.435 27.94) (width 1.75) (layer F.Cu) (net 9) (status 20))
 (segment (start 180.34 33.045) (end 180.34 29.845) (width 1.75) (layer F.Cu) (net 9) (status 10))
 (segment (start 180.58 55.245) (end 180.58 61.545) (width 1.75) (layer F.Cu) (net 11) (status 30))
 (segment (start 180.58 52.31) (end 178.435 50.165) (width 1.75) (layer F.Cu) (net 11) (status 20))
 (segment (start 180.58 55.245) (end 180.58 52.31) (width 1.75) (layer F.Cu) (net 11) (status 10))
 (segment (start 188.675 50.165) (end 196.215 42.625) (width 1.75) (layer F.Cu) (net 11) (status 20))
 (segment (start 178.435 50.165) (end 188.675 50.165) (width 1.75) (layer F.Cu) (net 11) (status 10))
 (segment (start 182.88 55.245) (end 183.515 55.245) (width 1.75) (layer F.Cu) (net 10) (status 30))
 (segment (start 188.595 55.245) (end 196.215 47.625) (width 1.75) (layer F.Cu) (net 10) (status 20))
 (segment (start 182.88 55.245) (end 188.595 55.245) (width 1.75) (layer F.Cu) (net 10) (status 10))
 (segment (start 173.79 61.595) (end 173.79 62.665) (width 1.75) (layer F.Cu) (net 10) (status 10))
 (segment (start 173.79 62.665) (end 175.26 64.135) (width 1.75) (layer F.Cu) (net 10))
 (segment (start 175.26 64.135) (end 183.515 64.135) (width 1.75) (layer F.Cu) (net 10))
 (segment (start 188.595 59.055) (end 188.595 55.245) (width 1.75) (layer F.Cu) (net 10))
 (segment (start 183.515 64.135) (end 188.595 59.055) (width 1.75) (layer F.Cu) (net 10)))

